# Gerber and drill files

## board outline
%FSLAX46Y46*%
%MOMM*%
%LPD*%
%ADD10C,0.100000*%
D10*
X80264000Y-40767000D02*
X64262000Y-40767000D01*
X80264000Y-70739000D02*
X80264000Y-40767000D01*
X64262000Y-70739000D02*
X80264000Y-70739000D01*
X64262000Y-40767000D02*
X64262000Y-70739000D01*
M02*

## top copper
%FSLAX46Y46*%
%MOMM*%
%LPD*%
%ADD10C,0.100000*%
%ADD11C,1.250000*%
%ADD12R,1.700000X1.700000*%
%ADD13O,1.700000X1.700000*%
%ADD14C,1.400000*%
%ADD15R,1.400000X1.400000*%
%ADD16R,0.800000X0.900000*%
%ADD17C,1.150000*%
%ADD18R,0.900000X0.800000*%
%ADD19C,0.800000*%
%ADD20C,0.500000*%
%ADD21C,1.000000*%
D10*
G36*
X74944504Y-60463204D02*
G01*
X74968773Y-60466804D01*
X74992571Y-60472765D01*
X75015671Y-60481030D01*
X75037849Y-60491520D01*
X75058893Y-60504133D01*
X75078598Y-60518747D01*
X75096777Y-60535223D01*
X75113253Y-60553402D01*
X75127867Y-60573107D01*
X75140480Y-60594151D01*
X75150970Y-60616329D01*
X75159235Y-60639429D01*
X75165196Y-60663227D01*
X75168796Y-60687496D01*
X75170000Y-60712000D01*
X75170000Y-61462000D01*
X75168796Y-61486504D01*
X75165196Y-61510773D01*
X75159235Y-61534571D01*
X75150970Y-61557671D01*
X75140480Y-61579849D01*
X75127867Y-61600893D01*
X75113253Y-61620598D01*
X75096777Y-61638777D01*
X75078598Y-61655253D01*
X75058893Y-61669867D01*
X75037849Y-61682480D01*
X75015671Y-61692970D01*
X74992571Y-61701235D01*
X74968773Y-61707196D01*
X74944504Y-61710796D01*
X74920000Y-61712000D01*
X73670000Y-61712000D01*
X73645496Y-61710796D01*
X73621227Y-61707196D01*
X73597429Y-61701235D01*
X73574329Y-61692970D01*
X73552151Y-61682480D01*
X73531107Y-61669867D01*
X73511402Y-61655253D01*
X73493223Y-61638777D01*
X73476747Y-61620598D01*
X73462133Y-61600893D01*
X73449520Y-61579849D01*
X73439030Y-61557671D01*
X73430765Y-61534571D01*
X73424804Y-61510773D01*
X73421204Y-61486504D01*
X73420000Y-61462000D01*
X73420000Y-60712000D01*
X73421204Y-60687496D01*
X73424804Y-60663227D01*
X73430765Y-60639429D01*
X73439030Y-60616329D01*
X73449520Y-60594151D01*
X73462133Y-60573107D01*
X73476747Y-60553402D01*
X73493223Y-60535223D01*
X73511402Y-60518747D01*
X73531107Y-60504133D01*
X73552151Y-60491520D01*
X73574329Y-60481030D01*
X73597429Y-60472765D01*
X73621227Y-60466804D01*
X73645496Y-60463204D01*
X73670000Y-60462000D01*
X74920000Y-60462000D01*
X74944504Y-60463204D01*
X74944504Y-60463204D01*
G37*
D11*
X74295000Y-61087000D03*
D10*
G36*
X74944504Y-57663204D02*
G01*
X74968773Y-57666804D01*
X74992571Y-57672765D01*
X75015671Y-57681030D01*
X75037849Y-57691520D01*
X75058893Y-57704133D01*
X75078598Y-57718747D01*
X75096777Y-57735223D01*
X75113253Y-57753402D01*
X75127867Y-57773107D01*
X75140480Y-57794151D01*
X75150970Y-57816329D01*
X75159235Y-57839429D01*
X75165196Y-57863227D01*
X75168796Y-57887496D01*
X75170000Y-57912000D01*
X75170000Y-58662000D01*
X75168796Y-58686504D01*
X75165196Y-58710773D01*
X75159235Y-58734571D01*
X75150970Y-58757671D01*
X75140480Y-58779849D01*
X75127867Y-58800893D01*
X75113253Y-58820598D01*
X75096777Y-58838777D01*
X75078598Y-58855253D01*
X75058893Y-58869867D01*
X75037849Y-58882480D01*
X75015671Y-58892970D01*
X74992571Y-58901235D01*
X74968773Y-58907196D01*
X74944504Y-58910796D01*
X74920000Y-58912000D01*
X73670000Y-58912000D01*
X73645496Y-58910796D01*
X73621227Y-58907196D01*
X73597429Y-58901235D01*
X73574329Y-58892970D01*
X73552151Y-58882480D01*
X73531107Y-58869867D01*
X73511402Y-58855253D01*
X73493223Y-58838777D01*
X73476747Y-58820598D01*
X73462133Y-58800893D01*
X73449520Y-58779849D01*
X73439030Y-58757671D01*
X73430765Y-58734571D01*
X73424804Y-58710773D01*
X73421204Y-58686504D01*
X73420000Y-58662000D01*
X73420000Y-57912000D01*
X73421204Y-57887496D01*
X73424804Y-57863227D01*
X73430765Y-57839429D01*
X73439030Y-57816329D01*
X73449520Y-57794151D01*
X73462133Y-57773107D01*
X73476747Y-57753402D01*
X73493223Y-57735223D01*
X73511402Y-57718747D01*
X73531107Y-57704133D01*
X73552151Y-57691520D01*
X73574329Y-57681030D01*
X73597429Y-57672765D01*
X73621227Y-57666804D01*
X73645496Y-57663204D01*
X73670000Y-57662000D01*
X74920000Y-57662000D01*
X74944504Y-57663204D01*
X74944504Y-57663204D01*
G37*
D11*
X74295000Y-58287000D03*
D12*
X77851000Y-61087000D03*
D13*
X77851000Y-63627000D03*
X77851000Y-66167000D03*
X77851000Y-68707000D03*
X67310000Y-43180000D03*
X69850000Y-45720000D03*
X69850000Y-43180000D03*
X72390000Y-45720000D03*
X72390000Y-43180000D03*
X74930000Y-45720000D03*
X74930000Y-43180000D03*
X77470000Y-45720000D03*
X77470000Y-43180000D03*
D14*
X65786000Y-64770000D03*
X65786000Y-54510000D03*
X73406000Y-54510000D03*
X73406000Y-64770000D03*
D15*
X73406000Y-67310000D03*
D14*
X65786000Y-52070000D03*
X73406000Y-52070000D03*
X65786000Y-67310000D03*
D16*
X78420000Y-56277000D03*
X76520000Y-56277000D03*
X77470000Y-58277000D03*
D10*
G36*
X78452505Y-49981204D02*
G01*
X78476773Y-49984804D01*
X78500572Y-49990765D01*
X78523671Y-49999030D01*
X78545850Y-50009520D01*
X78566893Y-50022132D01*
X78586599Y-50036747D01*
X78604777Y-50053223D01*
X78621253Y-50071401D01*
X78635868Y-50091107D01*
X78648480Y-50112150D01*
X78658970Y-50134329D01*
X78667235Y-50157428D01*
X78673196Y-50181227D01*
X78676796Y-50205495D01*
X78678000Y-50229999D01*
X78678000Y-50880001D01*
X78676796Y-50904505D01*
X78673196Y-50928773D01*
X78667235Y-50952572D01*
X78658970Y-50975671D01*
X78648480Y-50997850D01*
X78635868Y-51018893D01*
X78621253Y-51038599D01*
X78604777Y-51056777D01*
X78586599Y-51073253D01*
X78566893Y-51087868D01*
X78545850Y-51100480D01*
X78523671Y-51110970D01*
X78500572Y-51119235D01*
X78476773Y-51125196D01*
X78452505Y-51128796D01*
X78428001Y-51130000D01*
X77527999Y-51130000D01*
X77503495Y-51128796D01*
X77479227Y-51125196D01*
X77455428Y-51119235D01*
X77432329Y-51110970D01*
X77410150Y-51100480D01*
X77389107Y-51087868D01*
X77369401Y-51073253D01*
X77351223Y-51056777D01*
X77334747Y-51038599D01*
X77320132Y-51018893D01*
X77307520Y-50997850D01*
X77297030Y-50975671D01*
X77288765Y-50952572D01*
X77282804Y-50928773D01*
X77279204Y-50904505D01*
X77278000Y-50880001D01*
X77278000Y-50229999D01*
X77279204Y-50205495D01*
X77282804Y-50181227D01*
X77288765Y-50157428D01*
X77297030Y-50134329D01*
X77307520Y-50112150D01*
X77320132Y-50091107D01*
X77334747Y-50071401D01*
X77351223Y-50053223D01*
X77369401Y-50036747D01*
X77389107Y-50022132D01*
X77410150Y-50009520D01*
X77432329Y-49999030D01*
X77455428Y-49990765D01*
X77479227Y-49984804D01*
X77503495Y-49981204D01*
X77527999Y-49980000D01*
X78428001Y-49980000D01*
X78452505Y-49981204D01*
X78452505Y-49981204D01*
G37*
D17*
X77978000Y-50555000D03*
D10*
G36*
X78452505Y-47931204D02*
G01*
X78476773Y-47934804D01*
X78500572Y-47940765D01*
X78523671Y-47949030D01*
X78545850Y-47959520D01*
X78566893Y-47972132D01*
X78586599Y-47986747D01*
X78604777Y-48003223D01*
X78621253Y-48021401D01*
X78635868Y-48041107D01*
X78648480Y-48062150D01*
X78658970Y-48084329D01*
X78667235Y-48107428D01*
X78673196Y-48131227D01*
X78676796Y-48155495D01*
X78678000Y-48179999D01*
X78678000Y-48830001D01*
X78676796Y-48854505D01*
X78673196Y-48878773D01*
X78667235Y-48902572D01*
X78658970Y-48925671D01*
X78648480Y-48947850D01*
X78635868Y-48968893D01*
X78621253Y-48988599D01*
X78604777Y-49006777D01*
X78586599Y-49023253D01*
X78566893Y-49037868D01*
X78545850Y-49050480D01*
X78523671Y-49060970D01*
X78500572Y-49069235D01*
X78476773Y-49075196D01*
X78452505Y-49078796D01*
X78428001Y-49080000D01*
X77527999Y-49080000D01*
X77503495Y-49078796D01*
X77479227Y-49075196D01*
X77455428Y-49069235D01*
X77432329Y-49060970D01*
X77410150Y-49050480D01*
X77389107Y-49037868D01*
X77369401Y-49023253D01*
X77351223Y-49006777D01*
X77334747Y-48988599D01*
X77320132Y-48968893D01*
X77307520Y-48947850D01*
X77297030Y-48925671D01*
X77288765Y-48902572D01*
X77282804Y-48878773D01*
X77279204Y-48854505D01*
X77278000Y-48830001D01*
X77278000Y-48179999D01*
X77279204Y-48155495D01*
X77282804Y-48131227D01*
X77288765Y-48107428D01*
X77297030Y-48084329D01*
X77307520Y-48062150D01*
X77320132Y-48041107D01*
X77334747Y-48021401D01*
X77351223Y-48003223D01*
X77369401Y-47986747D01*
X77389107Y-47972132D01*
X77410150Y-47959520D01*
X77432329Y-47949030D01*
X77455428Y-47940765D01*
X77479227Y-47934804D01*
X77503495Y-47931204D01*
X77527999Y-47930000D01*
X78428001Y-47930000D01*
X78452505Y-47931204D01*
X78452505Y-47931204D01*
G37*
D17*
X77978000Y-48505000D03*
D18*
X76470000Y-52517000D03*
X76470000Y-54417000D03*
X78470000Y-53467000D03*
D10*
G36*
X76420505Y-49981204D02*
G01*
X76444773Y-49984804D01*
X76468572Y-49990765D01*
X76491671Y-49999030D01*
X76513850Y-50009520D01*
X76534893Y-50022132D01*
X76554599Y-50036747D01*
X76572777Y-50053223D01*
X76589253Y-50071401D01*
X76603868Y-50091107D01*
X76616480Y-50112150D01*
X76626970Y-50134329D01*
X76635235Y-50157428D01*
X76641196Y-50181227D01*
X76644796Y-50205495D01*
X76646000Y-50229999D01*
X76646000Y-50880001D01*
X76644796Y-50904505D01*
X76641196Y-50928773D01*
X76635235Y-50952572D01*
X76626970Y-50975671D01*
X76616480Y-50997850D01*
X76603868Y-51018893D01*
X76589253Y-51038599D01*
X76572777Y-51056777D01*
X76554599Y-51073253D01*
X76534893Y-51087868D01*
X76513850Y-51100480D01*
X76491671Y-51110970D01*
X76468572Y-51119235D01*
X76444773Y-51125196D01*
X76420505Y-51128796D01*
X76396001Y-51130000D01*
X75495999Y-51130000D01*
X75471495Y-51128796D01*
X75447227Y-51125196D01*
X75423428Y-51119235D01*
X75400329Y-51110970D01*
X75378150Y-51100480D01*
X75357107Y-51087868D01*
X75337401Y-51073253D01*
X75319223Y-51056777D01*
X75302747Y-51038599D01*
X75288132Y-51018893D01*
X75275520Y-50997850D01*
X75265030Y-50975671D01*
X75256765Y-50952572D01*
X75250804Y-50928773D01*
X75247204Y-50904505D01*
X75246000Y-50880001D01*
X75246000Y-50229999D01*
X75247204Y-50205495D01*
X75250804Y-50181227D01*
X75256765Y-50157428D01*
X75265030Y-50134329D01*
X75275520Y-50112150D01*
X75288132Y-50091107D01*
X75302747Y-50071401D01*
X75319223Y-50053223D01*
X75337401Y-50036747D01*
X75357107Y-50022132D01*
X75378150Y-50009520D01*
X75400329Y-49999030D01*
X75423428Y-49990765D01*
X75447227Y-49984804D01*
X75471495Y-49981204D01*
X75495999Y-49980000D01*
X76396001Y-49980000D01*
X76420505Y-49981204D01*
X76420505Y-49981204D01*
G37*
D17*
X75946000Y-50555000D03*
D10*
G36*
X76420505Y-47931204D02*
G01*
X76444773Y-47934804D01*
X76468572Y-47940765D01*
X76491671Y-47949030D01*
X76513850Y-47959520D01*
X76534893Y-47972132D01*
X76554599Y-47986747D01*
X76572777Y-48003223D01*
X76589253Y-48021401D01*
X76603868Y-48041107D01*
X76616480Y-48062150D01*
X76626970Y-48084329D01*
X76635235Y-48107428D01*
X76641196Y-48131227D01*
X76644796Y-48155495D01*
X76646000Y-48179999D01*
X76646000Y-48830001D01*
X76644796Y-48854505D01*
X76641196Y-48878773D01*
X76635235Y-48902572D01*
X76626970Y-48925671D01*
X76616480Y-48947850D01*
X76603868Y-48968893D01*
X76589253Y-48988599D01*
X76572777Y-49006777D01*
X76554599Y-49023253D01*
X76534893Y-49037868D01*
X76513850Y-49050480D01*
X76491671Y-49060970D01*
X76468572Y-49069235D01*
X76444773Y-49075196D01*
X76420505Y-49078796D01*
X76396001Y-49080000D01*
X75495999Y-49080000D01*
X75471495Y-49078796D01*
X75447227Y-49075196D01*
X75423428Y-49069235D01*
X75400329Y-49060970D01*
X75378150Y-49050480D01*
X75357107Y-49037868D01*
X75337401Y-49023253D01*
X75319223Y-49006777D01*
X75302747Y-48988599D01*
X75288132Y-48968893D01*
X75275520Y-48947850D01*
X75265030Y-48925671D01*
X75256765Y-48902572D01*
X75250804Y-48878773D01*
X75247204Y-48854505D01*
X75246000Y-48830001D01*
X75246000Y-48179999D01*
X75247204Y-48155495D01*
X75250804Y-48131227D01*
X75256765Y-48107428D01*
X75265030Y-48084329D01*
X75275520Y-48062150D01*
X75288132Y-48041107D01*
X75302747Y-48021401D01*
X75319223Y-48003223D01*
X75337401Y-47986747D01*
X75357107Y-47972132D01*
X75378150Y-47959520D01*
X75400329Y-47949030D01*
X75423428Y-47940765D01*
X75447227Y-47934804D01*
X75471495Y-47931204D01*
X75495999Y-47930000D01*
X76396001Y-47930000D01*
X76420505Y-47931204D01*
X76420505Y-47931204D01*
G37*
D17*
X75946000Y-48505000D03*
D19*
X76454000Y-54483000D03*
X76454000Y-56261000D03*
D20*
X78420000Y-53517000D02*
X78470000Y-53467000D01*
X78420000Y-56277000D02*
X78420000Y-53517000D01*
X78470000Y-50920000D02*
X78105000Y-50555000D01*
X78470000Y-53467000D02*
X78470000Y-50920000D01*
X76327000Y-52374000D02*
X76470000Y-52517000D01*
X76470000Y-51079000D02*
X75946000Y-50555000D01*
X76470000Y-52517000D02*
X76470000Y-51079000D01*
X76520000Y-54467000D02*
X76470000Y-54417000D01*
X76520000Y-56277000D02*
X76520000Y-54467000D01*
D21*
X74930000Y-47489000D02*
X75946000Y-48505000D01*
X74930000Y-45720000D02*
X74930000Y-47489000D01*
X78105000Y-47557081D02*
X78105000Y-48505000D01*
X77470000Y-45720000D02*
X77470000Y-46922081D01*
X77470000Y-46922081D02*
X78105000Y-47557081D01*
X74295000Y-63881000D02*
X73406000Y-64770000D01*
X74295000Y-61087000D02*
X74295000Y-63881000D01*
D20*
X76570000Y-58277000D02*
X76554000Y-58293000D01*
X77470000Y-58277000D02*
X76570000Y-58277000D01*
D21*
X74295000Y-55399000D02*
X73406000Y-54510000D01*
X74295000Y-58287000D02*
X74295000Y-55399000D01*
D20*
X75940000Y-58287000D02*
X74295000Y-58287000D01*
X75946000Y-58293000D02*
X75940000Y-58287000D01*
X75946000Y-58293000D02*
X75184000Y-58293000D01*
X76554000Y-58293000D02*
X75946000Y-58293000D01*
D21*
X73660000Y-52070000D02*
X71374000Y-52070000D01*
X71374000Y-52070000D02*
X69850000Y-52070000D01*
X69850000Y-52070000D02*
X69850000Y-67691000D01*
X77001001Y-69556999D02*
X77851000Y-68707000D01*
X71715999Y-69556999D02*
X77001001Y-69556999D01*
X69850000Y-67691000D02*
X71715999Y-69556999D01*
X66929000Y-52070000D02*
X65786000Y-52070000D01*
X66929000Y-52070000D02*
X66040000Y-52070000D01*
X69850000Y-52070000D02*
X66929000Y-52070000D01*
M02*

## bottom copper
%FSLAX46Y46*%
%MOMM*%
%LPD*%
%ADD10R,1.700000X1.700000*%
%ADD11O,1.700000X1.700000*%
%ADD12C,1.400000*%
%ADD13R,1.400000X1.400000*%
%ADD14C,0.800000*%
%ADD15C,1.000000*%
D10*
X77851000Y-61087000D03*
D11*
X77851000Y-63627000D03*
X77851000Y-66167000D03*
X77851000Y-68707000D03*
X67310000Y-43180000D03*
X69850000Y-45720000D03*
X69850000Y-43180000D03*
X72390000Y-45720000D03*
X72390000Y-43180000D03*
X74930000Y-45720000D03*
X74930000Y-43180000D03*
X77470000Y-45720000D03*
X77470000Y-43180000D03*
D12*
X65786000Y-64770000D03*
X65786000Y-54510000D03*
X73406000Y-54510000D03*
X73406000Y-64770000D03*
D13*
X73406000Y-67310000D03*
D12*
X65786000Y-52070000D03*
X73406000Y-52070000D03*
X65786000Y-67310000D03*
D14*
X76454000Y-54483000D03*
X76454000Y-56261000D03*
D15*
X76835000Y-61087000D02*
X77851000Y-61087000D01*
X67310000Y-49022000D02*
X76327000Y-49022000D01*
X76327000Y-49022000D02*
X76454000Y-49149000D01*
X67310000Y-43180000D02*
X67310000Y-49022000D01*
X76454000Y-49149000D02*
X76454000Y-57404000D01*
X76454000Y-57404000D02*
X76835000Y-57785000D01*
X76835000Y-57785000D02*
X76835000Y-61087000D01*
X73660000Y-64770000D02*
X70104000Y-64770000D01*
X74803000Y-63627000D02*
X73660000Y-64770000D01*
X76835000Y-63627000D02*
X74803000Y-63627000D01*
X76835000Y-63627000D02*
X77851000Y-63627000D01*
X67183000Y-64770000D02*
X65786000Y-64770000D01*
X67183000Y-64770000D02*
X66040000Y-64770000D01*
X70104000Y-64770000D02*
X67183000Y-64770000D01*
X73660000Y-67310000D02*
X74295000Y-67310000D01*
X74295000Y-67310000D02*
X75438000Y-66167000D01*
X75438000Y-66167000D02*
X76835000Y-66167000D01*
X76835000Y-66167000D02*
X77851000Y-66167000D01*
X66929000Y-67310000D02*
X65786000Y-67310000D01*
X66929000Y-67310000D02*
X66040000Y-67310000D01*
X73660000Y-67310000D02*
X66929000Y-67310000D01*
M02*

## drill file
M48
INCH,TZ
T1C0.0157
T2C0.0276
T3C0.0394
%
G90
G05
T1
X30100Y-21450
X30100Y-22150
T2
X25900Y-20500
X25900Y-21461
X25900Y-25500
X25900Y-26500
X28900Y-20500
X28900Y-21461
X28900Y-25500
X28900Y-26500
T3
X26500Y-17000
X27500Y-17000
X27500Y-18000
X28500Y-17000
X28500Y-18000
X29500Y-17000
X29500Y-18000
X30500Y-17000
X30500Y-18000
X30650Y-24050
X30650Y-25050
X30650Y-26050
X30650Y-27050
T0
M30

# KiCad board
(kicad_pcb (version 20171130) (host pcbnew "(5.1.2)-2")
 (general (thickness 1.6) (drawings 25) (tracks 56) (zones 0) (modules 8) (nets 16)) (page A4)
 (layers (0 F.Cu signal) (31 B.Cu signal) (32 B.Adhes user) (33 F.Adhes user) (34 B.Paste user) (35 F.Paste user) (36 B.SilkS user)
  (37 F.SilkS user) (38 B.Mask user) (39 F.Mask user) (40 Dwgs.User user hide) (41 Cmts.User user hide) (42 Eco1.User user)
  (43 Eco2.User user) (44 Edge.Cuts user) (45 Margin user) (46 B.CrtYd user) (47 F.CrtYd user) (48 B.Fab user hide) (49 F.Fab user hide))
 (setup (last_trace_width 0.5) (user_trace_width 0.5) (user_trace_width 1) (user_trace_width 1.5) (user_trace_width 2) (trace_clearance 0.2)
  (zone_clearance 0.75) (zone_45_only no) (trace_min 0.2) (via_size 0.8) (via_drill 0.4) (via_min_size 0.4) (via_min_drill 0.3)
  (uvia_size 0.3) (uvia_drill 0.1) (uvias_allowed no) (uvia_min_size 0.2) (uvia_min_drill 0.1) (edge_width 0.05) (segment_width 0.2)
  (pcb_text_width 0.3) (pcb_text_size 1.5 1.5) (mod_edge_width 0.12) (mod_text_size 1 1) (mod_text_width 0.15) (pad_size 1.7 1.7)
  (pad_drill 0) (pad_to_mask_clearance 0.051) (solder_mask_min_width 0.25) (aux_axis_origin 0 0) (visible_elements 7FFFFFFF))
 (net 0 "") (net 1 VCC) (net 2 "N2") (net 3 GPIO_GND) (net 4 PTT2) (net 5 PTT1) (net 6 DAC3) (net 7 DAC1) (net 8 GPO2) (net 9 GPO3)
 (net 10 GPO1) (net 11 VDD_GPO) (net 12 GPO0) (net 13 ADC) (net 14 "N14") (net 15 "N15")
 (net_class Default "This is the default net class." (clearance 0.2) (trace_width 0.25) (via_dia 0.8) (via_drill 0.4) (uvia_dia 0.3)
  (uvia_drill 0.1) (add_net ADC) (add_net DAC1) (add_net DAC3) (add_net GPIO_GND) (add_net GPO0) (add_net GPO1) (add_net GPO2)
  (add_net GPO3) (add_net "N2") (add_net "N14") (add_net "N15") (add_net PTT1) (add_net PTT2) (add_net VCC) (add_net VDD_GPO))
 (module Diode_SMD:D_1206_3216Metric (layer F.Cu) (at 74.295 59.687 90)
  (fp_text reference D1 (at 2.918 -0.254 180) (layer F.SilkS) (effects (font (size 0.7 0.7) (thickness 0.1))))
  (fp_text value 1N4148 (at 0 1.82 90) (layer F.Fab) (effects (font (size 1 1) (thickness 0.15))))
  (pad 1 smd roundrect (at -1.4 0 90) (size 1.25 1.75) (layers F.Cu F.Paste F.Mask) (roundrect_rratio 0.2) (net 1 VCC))
  (pad 2 smd roundrect (at 1.4 0 90) (size 1.25 1.75) (layers F.Cu F.Paste F.Mask) (roundrect_rratio 0.2) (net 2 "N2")))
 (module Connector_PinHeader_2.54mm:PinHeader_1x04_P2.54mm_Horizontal (layer F.Cu) (at 77.851 61.087)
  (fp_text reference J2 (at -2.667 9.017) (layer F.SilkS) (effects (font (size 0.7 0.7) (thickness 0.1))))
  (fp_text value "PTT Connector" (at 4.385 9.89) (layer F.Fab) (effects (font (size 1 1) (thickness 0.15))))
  (pad 1 thru_hole rect (at 0 0) (size 1.7 1.7) (drill 1) (layers *.Cu *.Mask) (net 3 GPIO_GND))
  (pad 2 thru_hole oval (at 0 2.54) (size 1.7 1.7) (drill 1) (layers *.Cu *.Mask) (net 1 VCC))
  (pad 3 thru_hole oval (at 0 5.08) (size 1.7 1.7) (drill 1) (layers *.Cu *.Mask) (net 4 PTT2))
  (pad 4 thru_hole oval (at 0 7.62) (size 1.7 1.7) (drill 1) (layers *.Cu *.Mask) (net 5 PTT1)))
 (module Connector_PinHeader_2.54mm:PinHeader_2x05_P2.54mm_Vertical (layer F.Cu) (at 67.31 45.72 90)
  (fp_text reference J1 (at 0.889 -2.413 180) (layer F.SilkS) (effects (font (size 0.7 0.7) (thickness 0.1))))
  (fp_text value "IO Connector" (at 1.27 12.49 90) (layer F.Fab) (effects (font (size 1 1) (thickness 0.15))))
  (pad 2 thru_hole oval (at 2.54 0 90) (size 1.7 1.7) (drill 1) (layers *.Cu *.Mask) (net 3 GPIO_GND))
  (pad 3 thru_hole oval (at 0 2.54 90) (size 1.7 1.7) (drill 1) (layers *.Cu *.Mask) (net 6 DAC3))
  (pad 4 thru_hole oval (at 2.54 2.54 90) (size 1.7 1.7) (drill 1) (layers *.Cu *.Mask) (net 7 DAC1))
  (pad 5 thru_hole oval (at 0 5.08 90) (size 1.7 1.7) (drill 1) (layers *.Cu *.Mask) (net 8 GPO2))
  (pad 6 thru_hole oval (at 2.54 5.08 90) (size 1.7 1.7) (drill 1) (layers *.Cu *.Mask) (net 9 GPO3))
  (pad 7 thru_hole oval (at 0 7.62 90) (size 1.7 1.7) (drill 1) (layers *.Cu *.Mask) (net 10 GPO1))
  (pad 8 thru_hole oval (at 2.54 7.62 90) (size 1.7 1.7) (drill 1) (layers *.Cu *.Mask) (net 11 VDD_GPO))
  (pad 9 thru_hole oval (at 0 10.16 90) (size 1.7 1.7) (drill 1) (layers *.Cu *.Mask) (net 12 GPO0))
  (pad 10 thru_hole oval (at 2.54 10.16 90) (size 1.7 1.7) (drill 1) (layers *.Cu *.Mask) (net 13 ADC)))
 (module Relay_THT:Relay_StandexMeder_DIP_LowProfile (layer F.Cu) (at 73.406 67.31 180)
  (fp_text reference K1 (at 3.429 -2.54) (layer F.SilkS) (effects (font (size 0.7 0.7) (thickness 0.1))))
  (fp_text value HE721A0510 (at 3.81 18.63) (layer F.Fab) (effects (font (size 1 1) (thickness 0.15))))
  (pad 13 thru_hole circle (at 7.62 2.54 180) (size 1.4 1.4) (drill 0.7) (layers *.Cu *.Mask) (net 1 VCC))
  (pad 9 thru_hole circle (at 7.62 12.8 180) (size 1.4 1.4) (drill 0.7) (layers *.Cu *.Mask))
  (pad 6 thru_hole circle (at 0 12.8 180) (size 1.4 1.4) (drill 0.7) (layers *.Cu *.Mask) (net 2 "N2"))
  (pad 2 thru_hole circle (at 0 2.54 180) (size 1.4 1.4) (drill 0.7) (layers *.Cu *.Mask) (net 1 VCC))
  (pad 1 thru_hole rect (at 0 0 180) (size 1.4 1.4) (drill 0.7) (layers *.Cu *.Mask) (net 4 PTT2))
  (pad 8 thru_hole circle (at 7.62 15.24 180) (size 1.4 1.4) (drill 0.7) (layers *.Cu *.Mask) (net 5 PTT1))
  (pad 7 thru_hole circle (at 0 15.24 180) (size 1.4 1.4) (drill 0.7) (layers *.Cu *.Mask) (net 5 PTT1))
  (pad 14 thru_hole circle (at 7.62 0 180) (size 1.4 1.4) (drill 0.7) (layers *.Cu *.Mask) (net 4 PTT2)))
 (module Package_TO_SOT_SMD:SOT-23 (layer F.Cu) (at 77.47 57.277 270)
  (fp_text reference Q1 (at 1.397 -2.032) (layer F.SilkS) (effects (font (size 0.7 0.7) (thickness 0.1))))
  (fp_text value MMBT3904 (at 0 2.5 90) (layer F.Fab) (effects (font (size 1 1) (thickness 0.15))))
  (pad 1 smd rect (at -1 -0.95 270) (size 0.9 0.8) (layers F.Cu F.Paste F.Mask) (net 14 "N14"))
  (pad 2 smd rect (at -1 0.95 270) (size 0.9 0.8) (layers F.Cu F.Paste F.Mask) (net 3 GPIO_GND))
  (pad 3 smd rect (at 1 0 270) (size 0.9 0.8) (layers F.Cu F.Paste F.Mask) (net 2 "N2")))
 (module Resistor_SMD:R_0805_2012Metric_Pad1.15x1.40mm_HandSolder (layer F.Cu) (at 77.978 49.53 90)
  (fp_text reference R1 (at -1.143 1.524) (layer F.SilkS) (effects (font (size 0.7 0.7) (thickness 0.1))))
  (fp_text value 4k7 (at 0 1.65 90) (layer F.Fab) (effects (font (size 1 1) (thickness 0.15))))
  (pad 1 smd roundrect (at -1.025 0 90) (size 1.15 1.4) (layers F.Cu F.Paste F.Mask) (roundrect_rratio 0.217391) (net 14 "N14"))
  (pad 2 smd roundrect (at 1.025 0 90) (size 1.15 1.4) (layers F.Cu F.Paste F.Mask) (roundrect_rratio 0.217391) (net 12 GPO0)))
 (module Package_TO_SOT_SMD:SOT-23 (layer F.Cu) (at 77.47 53.467)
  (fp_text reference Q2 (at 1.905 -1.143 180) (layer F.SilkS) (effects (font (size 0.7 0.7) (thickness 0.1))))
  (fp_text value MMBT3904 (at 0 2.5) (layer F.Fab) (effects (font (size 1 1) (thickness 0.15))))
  (pad 1 smd rect (at -1 -0.95) (size 0.9 0.8) (layers F.Cu F.Paste F.Mask) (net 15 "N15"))
  (pad 2 smd rect (at -1 0.95) (size 0.9 0.8) (layers F.Cu F.Paste F.Mask) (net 3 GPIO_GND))
  (pad 3 smd rect (at 1 0) (size 0.9 0.8) (layers F.Cu F.Paste F.Mask) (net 14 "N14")))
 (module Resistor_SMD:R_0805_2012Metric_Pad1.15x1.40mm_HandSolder (layer F.Cu) (at 75.946 49.53 90)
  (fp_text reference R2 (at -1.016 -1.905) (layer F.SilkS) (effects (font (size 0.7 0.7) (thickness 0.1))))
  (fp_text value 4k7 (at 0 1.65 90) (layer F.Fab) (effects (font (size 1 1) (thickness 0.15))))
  (pad 1 smd roundrect (at -1.025 0 90) (size 1.15 1.4) (layers F.Cu F.Paste F.Mask) (roundrect_rratio 0.217391) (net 15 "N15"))
  (pad 2 smd roundrect (at 1.025 0 90) (size 1.15 1.4) (layers F.Cu F.Paste F.Mask) (roundrect_rratio 0.217391) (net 10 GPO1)))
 (gr_line (start 80.264 40.767) (end 64.262 40.767) (layer Edge.Cuts) (width 0.1))
 (gr_line (start 80.264 70.739) (end 80.264 40.767) (layer Edge.Cuts) (width 0.1))
 (gr_line (start 64.262 70.739) (end 80.264 70.739) (layer Edge.Cuts) (width 0.1))
 (gr_line (start 64.262 40.767) (end 64.262 70.739) (layer Edge.Cuts) (width 0.1))
 (segment (start 78.42 53.517) (end 78.47 53.467) (width 0.5) (layer F.Cu) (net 14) (status 30))
 (segment (start 78.42 56.277) (end 78.42 53.517) (width 0.5) (layer F.Cu) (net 14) (status 30))
 (segment (start 78.47 50.92) (end 78.105 50.555) (width 0.5) (layer F.Cu) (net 14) (status 30))
 (segment (start 78.47 53.467) (end 78.47 50.92) (width 0.5) (layer F.Cu) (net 14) (status 30))
 (segment (start 76.327 52.374) (end 76.47 52.517) (width 0.5) (layer F.Cu) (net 15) (status 30))
 (segment (start 76.47 51.079) (end 75.946 50.555) (width 0.5) (layer F.Cu) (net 15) (status 30))
 (segment (start 76.47 52.517) (end 76.47 51.079) (width 0.5) (layer F.Cu) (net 15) (status 30))
 (via (at 76.454 54.483) (size 0.8) (drill 0.4) (layers F.Cu B.Cu) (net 3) (status 30))
 (segment (start 76.52 54.467) (end 76.47 54.417) (width 0.5) (layer F.Cu) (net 3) (status 30))
 (segment (start 76.52 56.277) (end 76.52 54.467) (width 0.5) (layer F.Cu) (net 3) (status 30))
 (via (at 76.454 56.261) (size 0.8) (drill 0.4) (layers F.Cu B.Cu) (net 3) (status 30))
 (segment (start 76.835 61.087) (end 77.851 61.087) (width 1) (layer B.Cu) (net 3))
 (segment (start 67.31 49.022) (end 76.327 49.022) (width 1) (layer B.Cu) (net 3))
 (segment (start 76.327 49.022) (end 76.454 49.149) (width 1) (layer B.Cu) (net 3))
 (segment (start 67.31 43.18) (end 67.31 49.022) (width 1) (layer B.Cu) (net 3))
 (segment (start 76.454 49.149) (end 76.454 57.404) (width 1) (layer B.Cu) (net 3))
 (segment (start 76.454 57.404) (end 76.835 57.785) (width 1) (layer B.Cu) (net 3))
 (segment (start 76.835 57.785) (end 76.835 61.087) (width 1) (layer B.Cu) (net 3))
 (segment (start 74.93 47.489) (end 75.946 48.505) (width 1) (layer F.Cu) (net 10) (status 20))
 (segment (start 74.93 45.72) (end 74.93 47.489) (width 1) (layer F.Cu) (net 10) (status 10))
 (segment (start 78.105 47.557081) (end 78.105 48.505) (width 1) (layer F.Cu) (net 12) (status 20))
 (segment (start 77.47 45.72) (end 77.47 46.922081) (width 1) (layer F.Cu) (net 12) (status 10))
 (segment (start 77.47 46.922081) (end 78.105 47.557081) (width 1) (layer F.Cu) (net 12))
 (segment (start 73.66 64.77) (end 70.104 64.77) (width 1) (layer B.Cu) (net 1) (status 10))
 (segment (start 74.803 63.627) (end 73.66 64.77) (width 1) (layer B.Cu) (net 1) (status 20))
 (segment (start 76.835 63.627) (end 74.803 63.627) (width 1) (layer B.Cu) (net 1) (status 10))
 (segment (start 76.835 63.627) (end 77.851 63.627) (width 1) (layer B.Cu) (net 1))
 (segment (start 67.183 64.77) (end 65.786 64.77) (width 1) (layer B.Cu) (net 1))
 (segment (start 67.183 64.77) (end 66.04 64.77) (width 1) (layer B.Cu) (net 1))
 (segment (start 70.104 64.77) (end 67.183 64.77) (width 1) (layer B.Cu) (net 1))
 (segment (start 74.295 63.881) (end 73.406 64.77) (width 1) (layer F.Cu) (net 1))
 (segment (start 74.295 61.087) (end 74.295 63.881) (width 1) (layer F.Cu) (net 1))
 (segment (start 76.57 58.277) (end 76.554 58.293) (width 0.5) (layer F.Cu) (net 2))
 (segment (start 77.47 58.277) (end 76.57 58.277) (width 0.5) (layer F.Cu) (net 2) (status 10))
 (segment (start 74.295 55.399) (end 73.406 54.51) (width 1) (layer F.Cu) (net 2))
 (segment (start 74.295 58.287) (end 74.295 55.399) (width 1) (layer F.Cu) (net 2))
 (segment (start 75.94 58.287) (end 74.295 58.287) (width 0.5) (layer F.Cu) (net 2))
 (segment (start 75.946 58.293) (end 75.94 58.287) (width 0.5) (layer F.Cu) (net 2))
 (segment (start 75.946 58.293) (end 75.184 58.293) (width 0.5) (layer F.Cu) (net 2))
 (segment (start 76.554 58.293) (end 75.946 58.293) (width 0.5) (layer F.Cu) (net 2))
 (segment (start 73.66 67.31) (end 74.295 67.31) (width 1) (layer B.Cu) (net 4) (status 30))
 (segment (start 74.295 67.31) (end 75.438 66.167) (width 1) (layer B.Cu) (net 4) (status 10))
 (segment (start 75.438 66.167) (end 76.835 66.167) (width 1) (layer B.Cu) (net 4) (status 20))
 (segment (start 76.835 66.167) (end 77.851 66.167) (width 1) (layer B.Cu) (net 4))
 (segment (start 66.929 67.31) (end 65.786 67.31) (width 1) (layer B.Cu) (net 4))
 (segment (start 66.929 67.31) (end 66.04 67.31) (width 1) (layer B.Cu) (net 4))
 (segment (start 73.66 67.31) (end 66.929 67.31) (width 1) (layer B.Cu) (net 4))
 (segment (start 73.66 52.07) (end 71.374 52.07) (width 1) (layer F.Cu) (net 5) (status 10))
 (segment (start 71.374 52.07) (end 69.85 52.07) (width 1) (layer F.Cu) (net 5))
 (segment (start 69.85 52.07) (end 69.85 67.691) (width 1) (layer F.Cu) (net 5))
 (segment (start 77.001001 69.556999) (end 77.851 68.707) (width 1) (layer F.Cu) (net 5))
 (segment (start 71.715999 69.556999) (end 77.001001 69.556999) (width 1) (layer F.Cu) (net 5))
 (segment (start 69.85 67.691) (end 71.715999 69.556999) (width 1) (layer F.Cu) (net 5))
 (segment (start 66.929 52.07) (end 65.786 52.07) (width 1) (layer F.Cu) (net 5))
 (segment (start 66.929 52.07) (end 66.04 52.07) (width 1) (layer F.Cu) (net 5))
 (segment (start 69.85 52.07) (end 66.929 52.07) (width 1) (layer F.Cu) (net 5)))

